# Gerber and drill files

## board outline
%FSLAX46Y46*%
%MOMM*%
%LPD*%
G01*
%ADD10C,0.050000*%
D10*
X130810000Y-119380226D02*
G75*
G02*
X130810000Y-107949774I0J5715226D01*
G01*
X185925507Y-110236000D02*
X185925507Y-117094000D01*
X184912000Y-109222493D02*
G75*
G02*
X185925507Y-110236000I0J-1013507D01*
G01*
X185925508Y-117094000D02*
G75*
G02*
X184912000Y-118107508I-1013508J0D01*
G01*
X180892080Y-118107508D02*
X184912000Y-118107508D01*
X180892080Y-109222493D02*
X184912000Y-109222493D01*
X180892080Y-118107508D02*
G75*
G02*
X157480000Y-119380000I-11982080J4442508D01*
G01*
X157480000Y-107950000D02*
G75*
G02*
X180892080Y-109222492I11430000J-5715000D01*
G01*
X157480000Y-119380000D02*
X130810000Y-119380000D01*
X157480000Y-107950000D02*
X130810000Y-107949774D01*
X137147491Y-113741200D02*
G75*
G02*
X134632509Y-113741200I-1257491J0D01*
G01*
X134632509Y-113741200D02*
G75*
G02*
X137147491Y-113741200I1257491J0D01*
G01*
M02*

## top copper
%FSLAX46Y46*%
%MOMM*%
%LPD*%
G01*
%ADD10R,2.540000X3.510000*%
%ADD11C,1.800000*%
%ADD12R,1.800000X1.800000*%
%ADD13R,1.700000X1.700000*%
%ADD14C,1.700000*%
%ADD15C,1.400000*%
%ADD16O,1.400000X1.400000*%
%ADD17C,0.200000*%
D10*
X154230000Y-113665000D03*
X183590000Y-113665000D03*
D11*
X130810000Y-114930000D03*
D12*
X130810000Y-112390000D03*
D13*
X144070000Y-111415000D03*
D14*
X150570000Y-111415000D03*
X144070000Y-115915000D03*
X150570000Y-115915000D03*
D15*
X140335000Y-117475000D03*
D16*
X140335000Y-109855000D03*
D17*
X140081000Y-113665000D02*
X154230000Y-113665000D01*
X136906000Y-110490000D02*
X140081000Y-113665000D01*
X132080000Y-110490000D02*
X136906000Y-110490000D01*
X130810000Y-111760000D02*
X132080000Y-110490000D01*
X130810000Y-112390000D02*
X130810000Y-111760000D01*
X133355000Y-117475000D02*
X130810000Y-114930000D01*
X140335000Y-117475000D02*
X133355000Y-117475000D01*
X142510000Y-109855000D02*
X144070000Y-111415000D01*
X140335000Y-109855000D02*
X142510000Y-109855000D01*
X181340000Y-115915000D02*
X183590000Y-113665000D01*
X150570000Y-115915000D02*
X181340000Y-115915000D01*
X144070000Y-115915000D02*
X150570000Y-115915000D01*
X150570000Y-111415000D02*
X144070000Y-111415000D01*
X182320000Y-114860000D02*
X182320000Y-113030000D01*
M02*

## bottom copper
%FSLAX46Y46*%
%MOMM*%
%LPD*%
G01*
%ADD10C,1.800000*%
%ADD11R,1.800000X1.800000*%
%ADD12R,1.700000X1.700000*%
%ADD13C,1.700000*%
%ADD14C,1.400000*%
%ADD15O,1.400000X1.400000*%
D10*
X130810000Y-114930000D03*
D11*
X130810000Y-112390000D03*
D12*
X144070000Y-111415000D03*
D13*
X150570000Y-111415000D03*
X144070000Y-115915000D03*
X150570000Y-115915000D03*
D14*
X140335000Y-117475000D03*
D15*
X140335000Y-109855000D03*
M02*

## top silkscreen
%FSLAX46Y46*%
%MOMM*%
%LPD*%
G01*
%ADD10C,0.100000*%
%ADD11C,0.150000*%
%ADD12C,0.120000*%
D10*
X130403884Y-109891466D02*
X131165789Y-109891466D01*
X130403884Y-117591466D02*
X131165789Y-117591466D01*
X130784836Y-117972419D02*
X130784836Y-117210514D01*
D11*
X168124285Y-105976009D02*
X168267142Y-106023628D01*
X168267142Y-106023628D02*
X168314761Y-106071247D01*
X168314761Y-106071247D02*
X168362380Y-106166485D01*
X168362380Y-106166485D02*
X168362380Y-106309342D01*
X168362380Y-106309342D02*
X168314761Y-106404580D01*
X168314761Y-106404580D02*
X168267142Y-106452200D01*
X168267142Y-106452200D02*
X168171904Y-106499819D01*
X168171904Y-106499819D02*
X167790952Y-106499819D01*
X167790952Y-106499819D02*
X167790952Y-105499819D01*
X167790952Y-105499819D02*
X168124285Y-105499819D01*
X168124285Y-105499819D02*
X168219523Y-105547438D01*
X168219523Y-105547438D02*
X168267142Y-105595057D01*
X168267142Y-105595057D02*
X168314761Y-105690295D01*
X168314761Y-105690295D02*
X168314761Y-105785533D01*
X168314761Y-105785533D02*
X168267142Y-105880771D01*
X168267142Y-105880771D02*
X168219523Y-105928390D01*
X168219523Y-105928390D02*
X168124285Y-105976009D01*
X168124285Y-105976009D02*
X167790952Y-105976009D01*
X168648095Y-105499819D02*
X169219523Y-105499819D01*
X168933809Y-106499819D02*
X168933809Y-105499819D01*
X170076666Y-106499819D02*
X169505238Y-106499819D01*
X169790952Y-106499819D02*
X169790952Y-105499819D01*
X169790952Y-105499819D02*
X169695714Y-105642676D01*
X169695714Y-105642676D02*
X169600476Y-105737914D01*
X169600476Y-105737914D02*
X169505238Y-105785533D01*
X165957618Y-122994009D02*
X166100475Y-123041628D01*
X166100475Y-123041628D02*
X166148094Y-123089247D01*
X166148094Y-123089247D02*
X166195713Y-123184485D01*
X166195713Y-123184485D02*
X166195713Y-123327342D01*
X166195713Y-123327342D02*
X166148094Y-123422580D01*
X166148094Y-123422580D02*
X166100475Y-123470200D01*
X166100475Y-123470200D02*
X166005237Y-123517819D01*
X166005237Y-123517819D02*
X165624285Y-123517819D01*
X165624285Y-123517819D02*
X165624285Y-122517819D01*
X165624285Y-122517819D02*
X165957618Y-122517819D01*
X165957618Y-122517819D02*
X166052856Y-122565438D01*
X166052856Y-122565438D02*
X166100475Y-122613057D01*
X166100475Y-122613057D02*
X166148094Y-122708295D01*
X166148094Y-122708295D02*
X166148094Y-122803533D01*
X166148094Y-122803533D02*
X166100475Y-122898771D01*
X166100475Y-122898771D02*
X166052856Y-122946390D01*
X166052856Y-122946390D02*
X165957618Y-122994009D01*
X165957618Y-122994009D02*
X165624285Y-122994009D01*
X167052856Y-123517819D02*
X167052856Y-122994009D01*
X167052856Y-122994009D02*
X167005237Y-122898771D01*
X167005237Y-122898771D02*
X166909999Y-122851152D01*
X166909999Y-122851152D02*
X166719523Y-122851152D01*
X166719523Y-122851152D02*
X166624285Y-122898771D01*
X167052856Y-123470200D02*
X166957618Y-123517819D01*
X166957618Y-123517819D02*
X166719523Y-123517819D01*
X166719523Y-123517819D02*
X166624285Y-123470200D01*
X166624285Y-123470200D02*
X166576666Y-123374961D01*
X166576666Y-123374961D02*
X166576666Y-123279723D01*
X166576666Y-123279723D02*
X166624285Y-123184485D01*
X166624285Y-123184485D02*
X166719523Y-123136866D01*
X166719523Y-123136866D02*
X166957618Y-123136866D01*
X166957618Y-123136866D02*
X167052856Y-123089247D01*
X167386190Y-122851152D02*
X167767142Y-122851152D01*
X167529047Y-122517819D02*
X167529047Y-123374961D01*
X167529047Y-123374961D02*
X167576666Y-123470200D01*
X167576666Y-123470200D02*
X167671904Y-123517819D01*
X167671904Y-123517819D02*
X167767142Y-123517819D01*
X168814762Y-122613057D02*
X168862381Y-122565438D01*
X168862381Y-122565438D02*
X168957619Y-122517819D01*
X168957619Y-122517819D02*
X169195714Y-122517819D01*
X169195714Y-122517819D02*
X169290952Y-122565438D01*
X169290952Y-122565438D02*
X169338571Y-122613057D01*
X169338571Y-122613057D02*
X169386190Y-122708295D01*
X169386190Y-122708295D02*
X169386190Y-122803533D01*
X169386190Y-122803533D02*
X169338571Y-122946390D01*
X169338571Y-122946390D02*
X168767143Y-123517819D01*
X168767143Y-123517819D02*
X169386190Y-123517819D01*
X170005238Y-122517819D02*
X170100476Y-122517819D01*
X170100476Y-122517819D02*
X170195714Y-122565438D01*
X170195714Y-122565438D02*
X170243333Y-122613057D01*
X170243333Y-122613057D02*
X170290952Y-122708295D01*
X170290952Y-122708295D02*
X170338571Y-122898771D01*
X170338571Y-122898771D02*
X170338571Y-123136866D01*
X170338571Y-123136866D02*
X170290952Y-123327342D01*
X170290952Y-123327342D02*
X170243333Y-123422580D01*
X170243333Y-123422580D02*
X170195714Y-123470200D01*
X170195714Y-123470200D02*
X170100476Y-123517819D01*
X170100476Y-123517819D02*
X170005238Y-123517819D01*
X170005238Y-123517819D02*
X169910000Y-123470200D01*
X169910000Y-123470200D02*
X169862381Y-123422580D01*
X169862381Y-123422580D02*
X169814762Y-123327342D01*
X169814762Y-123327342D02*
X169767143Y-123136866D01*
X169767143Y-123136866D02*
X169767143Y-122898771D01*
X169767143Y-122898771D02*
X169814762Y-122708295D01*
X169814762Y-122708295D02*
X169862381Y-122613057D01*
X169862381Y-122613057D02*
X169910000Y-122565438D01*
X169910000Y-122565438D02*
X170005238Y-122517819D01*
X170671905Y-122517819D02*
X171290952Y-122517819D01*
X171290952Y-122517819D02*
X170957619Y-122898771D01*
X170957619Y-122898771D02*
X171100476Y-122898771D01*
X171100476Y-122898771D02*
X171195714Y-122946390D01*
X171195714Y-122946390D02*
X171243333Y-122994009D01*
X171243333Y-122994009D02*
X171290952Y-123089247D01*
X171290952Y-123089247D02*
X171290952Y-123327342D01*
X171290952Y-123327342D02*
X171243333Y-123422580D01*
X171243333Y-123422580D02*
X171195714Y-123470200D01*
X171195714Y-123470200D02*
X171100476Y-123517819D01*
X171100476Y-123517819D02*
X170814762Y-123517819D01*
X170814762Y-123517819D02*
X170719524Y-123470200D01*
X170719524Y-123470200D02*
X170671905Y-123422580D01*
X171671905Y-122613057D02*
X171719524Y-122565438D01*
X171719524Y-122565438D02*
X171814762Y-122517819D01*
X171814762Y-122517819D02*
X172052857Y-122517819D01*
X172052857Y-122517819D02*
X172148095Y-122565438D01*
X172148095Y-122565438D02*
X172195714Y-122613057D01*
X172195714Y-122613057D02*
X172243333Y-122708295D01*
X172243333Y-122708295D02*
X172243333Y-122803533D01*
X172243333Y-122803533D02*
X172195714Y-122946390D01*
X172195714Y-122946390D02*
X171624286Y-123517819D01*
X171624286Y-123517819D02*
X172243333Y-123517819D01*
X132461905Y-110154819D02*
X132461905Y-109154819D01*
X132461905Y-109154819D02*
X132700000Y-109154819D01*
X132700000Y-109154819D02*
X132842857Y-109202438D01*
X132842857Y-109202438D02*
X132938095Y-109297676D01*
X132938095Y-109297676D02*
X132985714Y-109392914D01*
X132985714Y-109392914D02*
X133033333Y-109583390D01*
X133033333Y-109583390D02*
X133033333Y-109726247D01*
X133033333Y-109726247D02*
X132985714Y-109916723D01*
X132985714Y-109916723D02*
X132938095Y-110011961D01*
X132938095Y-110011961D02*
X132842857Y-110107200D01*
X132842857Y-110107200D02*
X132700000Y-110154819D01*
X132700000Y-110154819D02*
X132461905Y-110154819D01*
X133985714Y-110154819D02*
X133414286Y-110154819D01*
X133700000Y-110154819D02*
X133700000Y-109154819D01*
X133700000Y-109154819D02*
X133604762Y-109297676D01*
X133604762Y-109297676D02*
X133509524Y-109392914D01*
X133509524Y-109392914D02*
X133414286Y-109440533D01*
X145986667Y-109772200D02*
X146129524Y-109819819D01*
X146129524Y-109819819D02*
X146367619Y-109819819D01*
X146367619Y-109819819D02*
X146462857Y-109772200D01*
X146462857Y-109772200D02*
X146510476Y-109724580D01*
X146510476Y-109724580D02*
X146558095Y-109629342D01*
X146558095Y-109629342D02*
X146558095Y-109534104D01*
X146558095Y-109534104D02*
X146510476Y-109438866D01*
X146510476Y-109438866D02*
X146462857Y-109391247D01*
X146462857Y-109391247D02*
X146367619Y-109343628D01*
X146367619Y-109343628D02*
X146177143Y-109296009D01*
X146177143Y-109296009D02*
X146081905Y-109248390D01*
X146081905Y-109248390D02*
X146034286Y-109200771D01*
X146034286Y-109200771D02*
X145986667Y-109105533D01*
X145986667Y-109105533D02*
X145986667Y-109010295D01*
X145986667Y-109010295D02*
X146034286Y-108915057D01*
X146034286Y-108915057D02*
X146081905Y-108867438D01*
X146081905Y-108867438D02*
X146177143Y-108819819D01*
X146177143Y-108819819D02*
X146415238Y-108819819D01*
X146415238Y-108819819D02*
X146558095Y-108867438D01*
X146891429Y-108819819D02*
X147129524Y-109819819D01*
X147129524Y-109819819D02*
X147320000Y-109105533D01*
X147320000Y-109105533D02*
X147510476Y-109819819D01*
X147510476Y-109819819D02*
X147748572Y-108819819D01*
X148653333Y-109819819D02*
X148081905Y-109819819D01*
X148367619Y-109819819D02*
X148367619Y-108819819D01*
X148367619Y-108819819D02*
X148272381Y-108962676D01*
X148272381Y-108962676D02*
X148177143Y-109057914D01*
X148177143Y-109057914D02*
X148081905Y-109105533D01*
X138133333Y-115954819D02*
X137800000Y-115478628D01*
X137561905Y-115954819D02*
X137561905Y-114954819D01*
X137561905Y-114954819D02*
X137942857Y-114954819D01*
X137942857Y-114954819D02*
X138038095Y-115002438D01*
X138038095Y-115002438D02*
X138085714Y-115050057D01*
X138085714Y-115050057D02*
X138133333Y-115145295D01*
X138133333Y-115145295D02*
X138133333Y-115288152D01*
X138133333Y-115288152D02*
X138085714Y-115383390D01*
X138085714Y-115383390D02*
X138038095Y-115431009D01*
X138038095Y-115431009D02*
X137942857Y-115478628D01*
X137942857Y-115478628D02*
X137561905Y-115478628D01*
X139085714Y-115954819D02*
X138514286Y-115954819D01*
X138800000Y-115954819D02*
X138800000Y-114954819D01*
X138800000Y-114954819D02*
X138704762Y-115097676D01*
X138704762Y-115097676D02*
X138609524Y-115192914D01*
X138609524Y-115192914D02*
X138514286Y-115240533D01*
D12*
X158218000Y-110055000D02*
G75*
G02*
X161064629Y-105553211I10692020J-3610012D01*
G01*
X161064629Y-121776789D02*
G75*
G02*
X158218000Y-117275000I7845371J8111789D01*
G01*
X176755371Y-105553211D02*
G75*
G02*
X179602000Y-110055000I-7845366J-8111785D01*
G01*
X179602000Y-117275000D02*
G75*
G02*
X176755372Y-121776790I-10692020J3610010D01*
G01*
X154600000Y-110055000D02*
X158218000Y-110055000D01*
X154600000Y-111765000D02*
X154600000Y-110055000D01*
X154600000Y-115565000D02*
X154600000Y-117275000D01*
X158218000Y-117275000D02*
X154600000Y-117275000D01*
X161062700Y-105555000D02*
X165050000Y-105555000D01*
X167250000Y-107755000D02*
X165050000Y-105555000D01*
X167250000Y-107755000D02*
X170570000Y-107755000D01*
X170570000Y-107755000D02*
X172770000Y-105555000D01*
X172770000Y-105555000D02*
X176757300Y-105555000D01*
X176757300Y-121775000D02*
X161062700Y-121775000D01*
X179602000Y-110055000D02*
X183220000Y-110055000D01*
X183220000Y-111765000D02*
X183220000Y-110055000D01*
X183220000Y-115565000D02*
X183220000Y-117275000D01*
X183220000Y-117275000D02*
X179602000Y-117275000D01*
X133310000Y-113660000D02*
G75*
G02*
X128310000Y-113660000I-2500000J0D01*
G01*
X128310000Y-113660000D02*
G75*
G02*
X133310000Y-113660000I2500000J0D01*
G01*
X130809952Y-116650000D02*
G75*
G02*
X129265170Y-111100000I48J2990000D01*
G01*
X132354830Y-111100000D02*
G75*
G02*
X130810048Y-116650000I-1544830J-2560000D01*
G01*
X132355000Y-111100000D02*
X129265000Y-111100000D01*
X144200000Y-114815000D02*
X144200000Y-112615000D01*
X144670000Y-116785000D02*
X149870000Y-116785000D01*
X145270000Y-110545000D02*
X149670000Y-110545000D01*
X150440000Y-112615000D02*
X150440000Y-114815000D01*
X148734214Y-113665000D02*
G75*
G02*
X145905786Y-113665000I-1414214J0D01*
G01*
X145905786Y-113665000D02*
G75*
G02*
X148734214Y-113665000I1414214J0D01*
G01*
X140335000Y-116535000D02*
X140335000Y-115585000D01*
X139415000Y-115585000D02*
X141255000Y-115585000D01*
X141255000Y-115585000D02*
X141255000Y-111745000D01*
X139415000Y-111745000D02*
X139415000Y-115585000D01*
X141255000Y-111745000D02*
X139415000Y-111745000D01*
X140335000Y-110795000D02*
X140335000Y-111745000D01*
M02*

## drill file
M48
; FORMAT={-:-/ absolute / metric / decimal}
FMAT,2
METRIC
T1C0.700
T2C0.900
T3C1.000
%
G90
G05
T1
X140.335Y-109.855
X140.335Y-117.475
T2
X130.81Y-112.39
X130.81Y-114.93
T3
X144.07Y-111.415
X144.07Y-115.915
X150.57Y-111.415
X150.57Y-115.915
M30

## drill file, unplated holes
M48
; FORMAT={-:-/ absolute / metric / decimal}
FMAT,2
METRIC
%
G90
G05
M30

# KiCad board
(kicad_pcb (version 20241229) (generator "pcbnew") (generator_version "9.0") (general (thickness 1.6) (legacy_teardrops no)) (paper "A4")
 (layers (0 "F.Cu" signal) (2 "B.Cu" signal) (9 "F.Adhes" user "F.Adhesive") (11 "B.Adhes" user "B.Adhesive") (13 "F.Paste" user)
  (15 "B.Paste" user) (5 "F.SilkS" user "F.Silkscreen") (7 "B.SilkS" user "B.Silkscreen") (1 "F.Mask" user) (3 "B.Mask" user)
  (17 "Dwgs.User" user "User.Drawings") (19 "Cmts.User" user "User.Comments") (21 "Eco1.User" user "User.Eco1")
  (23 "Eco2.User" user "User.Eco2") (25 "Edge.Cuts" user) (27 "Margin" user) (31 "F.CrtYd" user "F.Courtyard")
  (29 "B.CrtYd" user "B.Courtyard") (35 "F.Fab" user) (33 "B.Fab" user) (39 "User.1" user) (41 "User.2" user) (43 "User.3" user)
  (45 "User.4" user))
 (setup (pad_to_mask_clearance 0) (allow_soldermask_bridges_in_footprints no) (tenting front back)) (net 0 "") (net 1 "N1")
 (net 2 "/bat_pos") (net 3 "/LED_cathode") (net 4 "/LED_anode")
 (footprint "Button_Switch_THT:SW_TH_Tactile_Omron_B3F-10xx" (layer "F.Cu") (at 144.07 111.415)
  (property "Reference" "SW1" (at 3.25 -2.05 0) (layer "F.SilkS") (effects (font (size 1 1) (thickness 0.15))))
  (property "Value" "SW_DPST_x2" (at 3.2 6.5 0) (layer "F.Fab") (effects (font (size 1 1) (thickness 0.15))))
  (fp_line (start 0.13 3.4) (end 0.13 1.2) (stroke (width 0.12) (type solid)) (layer "F.SilkS"))
  (fp_line (start 0.6 5.37) (end 5.8 5.37) (stroke (width 0.12) (type solid)) (layer "F.SilkS"))
  (fp_line (start 1.2 -0.87) (end 5.6 -0.87) (stroke (width 0.12) (type solid)) (layer "F.SilkS"))
  (fp_line (start 6.37 1.2) (end 6.37 3.4) (stroke (width 0.12) (type solid)) (layer "F.SilkS"))
  (fp_circle (center 3.25 2.25) (end 4.25 3.25) (stroke (width 0.12) (type solid)) (fill no) (layer "F.SilkS"))
  (pad "1" thru_hole rect (at 0 0) (size 1.7 1.7) (drill 1) (layers "*.Cu" "*.Mask") (remove_unused_layers no) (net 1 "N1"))
  (pad "1" thru_hole circle (at 6.5 0) (size 1.7 1.7) (drill 1) (layers "*.Cu" "*.Mask") (remove_unused_layers no) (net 1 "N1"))
  (pad "2" thru_hole circle (at 0 4.5) (size 1.7 1.7) (drill 1) (layers "*.Cu" "*.Mask") (remove_unused_layers no) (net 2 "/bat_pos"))
  (pad "2" thru_hole circle (at 6.5 4.5) (size 1.7 1.7) (drill 1) (layers "*.Cu" "*.Mask") (remove_unused_layers no) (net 2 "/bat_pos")))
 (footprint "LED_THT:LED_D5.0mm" (layer "F.Cu") (at 130.81 112.39 -90)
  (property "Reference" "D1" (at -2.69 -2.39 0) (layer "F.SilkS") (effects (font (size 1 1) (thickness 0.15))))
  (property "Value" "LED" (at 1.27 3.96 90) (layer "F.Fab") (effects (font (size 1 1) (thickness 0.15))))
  (fp_line (start -1.29 -1.545) (end -1.29 1.545) (stroke (width 0.12) (type solid)) (layer "F.SilkS"))
  (fp_arc (start 4.26 0.000048) (mid 2.071756 2.880501) (end -1.29 1.54483) (stroke (width 0.12) (type solid)) (layer "F.SilkS"))
  (fp_arc (start -1.29 -1.54483) (mid 2.071756 -2.880501) (end 4.26 -0.000048) (stroke (width 0.12) (type solid)) (layer "F.SilkS"))
  (fp_circle (center 1.27 0) (end 3.77 0) (stroke (width 0.12) (type solid)) (fill no) (layer "F.SilkS"))
  (pad "1" thru_hole rect (at 0 0 270) (size 1.8 1.8) (drill 0.9) (layers "*.Cu" "*.Mask") (remove_unused_layers no) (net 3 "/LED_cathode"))
  (pad "2" thru_hole circle (at 2.54 0 270) (size 1.8 1.8) (drill 0.9) (layers "*.Cu" "*.Mask") (remove_unused_layers no)
   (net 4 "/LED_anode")))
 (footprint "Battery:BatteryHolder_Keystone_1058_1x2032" (layer "F.Cu") (at 168.91 113.665 180)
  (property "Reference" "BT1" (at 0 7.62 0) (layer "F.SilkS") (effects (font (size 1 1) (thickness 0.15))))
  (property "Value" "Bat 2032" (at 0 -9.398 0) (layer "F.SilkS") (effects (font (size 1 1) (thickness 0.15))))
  (fp_line (start 14.31 3.61) (end 10.692 3.61) (stroke (width 0.12) (type solid)) (layer "F.SilkS"))
  (fp_line (start 14.31 1.9) (end 14.31 3.61) (stroke (width 0.12) (type solid)) (layer "F.SilkS"))
  (fp_line (start 14.31 -1.9) (end 14.31 -3.61) (stroke (width 0.12) (type solid)) (layer "F.SilkS"))
  (fp_line (start 10.692 -3.61) (end 14.31 -3.61) (stroke (width 0.12) (type solid)) (layer "F.SilkS"))
  (fp_line (start 7.8473 8.11) (end 3.86 8.11) (stroke (width 0.12) (type solid)) (layer "F.SilkS"))
  (fp_line (start 1.66 5.91) (end 3.86 8.11) (stroke (width 0.12) (type solid)) (layer "F.SilkS"))
  (fp_line (start 1.66 5.91) (end -1.66 5.91) (stroke (width 0.12) (type solid)) (layer "F.SilkS"))
  (fp_line (start -1.66 5.91) (end -3.86 8.11) (stroke (width 0.12) (type solid)) (layer "F.SilkS"))
  (fp_line (start -3.86 8.11) (end -7.8473 8.11) (stroke (width 0.12) (type solid)) (layer "F.SilkS"))
  (fp_line (start -7.8473 -8.11) (end 7.8473 -8.11) (stroke (width 0.12) (type solid)) (layer "F.SilkS"))
  (fp_line (start -10.692 3.61) (end -14.31 3.61) (stroke (width 0.12) (type solid)) (layer "F.SilkS"))
  (fp_line (start -14.31 1.9) (end -14.31 3.61) (stroke (width 0.12) (type solid)) (layer "F.SilkS"))
  (fp_line (start -14.31 -1.9) (end -14.31 -3.61) (stroke (width 0.12) (type solid)) (layer "F.SilkS"))
  (fp_line (start -14.31 -3.61) (end -10.692 -3.61) (stroke (width 0.12) (type solid)) (layer "F.SilkS"))
  (fp_arc (start 10.692 3.61) (mid 9.538084 6.031244) (end 7.845371 8.111789) (stroke (width 0.12) (type solid)) (layer "F.SilkS"))
  (fp_arc (start 7.845371 -8.111789) (mid 9.538085 -6.031244) (end 10.692 -3.61) (stroke (width 0.12) (type solid)) (layer "F.SilkS"))
  (fp_arc (start -7.845371 8.111789) (mid -9.538085 6.031244) (end -10.692 3.61) (stroke (width 0.12) (type solid)) (layer "F.SilkS"))
  (fp_arc (start -10.692 -3.61) (mid -9.538084 -6.031244) (end -7.845371 -8.111789) (stroke (width 0.12) (type solid)) (layer "F.SilkS"))
  (pad "1" smd rect (at -14.68 0 180) (size 2.54 3.51) (layers "F.Cu" "F.Mask" "F.Paste") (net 2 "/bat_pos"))
  (pad "2" smd rect (at 14.68 0 180) (size 2.54 3.51) (layers "F.Cu" "F.Mask" "F.Paste") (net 3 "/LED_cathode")))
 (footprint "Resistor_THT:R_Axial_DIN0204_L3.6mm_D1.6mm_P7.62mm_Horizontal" (layer "F.Cu") (at 140.335 117.475 90)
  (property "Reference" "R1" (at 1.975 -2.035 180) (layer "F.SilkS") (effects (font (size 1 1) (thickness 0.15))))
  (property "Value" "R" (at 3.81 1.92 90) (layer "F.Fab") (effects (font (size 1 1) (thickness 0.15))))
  (fp_line (start 5.73 -0.92) (end 1.89 -0.92) (stroke (width 0.12) (type solid)) (layer "F.SilkS"))
  (fp_line (start 1.89 -0.92) (end 1.89 0.92) (stroke (width 0.12) (type solid)) (layer "F.SilkS"))
  (fp_line (start 6.68 0) (end 5.73 0) (stroke (width 0.12) (type solid)) (layer "F.SilkS"))
  (fp_line (start 0.94 0) (end 1.89 0) (stroke (width 0.12) (type solid)) (layer "F.SilkS"))
  (fp_line (start 5.73 0.92) (end 5.73 -0.92) (stroke (width 0.12) (type solid)) (layer "F.SilkS"))
  (fp_line (start 1.89 0.92) (end 5.73 0.92) (stroke (width 0.12) (type solid)) (layer "F.SilkS"))
  (pad "1" thru_hole circle (at 0 0 90) (size 1.4 1.4) (drill 0.7) (layers "*.Cu" "*.Mask") (remove_unused_layers no) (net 4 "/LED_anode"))
  (pad "2" thru_hole oval (at 7.62 0 90) (size 1.4 1.4) (drill 0.7) (layers "*.Cu" "*.Mask") (remove_unused_layers no) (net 1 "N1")))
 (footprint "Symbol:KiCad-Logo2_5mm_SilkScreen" (layer "B.Cu") (at 168.91 109.22 180)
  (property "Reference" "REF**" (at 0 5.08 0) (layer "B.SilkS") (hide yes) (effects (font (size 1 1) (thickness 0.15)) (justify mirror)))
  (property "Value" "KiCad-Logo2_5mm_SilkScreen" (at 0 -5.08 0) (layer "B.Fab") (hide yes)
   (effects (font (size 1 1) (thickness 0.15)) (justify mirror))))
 (gr_line (start 157.48 119.38) (end 130.81 119.38) (stroke (width 0.05) (type default)) (locked yes) (layer "Edge.Cuts"))
 (gr_arc (start 157.48 107.95) (mid 169.603547 100.904705) (end 180.89208 109.222492) (stroke (width 0.05) (type default)) (locked yes)
  (layer "Edge.Cuts"))
 (gr_arc (start 130.81 119.380226) (mid 125.094774 113.665) (end 130.81 107.949774) (stroke (width 0.05) (type default)) (locked yes)
  (layer "Edge.Cuts"))
 (gr_line (start 185.925507 110.236) (end 185.925507 117.094) (stroke (width 0.05) (type default)) (locked yes) (layer "Edge.Cuts"))
 (gr_arc (start 185.925508 117.094) (mid 185.628658 117.810658) (end 184.912 118.107508) (stroke (width 0.05) (type default)) (locked yes)
  (layer "Edge.Cuts"))
 (gr_arc (start 184.912 109.222493) (mid 185.628658 109.519342) (end 185.925507 110.236) (stroke (width 0.05) (type default)) (locked yes)
  (layer "Edge.Cuts"))
 (gr_circle (center 135.89 113.7412) (end 135.365754 114.8842) (stroke (width 0.05) (type default)) (fill no) (layer "Edge.Cuts"))
 (gr_line (start 180.89208 109.222493) (end 184.912 109.222493) (stroke (width 0.05) (type default)) (locked yes) (layer "Edge.Cuts"))
 (gr_line (start 157.48 107.95) (end 130.81 107.949774) (stroke (width 0.05) (type solid)) (locked yes) (layer "Edge.Cuts"))
 (gr_arc (start 180.89208 118.107508) (mid 169.603547 126.425294) (end 157.48 119.38) (stroke (width 0.05) (type default)) (locked yes)
  (layer "Edge.Cuts"))
 (gr_line (start 180.89208 118.107508) (end 184.912 118.107508) (stroke (width 0.05) (type default)) (locked yes) (layer "Edge.Cuts"))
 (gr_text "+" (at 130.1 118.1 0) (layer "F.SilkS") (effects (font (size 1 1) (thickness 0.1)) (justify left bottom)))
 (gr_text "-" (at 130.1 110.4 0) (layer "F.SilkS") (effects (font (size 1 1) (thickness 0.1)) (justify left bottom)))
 (segment (start 144.07 115.915) (end 150.57 115.915) (width 0.2) (layer "F.Cu") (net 2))
 (segment (start 150.57 115.915) (end 181.34 115.915) (width 0.2) (layer "F.Cu") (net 2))
 (segment (start 182.32 114.86) (end 182.32 113.03) (width 0.2) (layer "F.Cu") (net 2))
 (segment (start 181.34 115.915) (end 183.59 113.665) (width 0.2) (layer "F.Cu") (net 2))
 (segment (start 130.81 111.76) (end 132.08 110.49) (width 0.2) (layer "F.Cu") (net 3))
 (segment (start 132.08 110.49) (end 136.906 110.49) (width 0.2) (layer "F.Cu") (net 3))
 (segment (start 130.81 112.39) (end 130.81 111.76) (width 0.2) (layer "F.Cu") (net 3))
 (segment (start 140.081 113.665) (end 154.23 113.665) (width 0.2) (layer "F.Cu") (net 3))
 (segment (start 136.906 110.49) (end 140.081 113.665) (width 0.2) (layer "F.Cu") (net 3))
 (segment (start 140.335 117.475) (end 133.355 117.475) (width 0.2) (layer "F.Cu") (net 4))
 (segment (start 133.355 117.475) (end 130.81 114.93) (width 0.2) (layer "F.Cu") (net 4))
 (segment (start 142.51 109.855) (end 144.07 111.415) (width 0.2) (layer "F.Cu") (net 1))
 (segment (start 150.57 111.415) (end 144.07 111.415) (width 0.2) (layer "F.Cu") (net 1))
 (segment (start 140.335 109.855) (end 142.51 109.855) (width 0.2) (layer "F.Cu") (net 1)))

